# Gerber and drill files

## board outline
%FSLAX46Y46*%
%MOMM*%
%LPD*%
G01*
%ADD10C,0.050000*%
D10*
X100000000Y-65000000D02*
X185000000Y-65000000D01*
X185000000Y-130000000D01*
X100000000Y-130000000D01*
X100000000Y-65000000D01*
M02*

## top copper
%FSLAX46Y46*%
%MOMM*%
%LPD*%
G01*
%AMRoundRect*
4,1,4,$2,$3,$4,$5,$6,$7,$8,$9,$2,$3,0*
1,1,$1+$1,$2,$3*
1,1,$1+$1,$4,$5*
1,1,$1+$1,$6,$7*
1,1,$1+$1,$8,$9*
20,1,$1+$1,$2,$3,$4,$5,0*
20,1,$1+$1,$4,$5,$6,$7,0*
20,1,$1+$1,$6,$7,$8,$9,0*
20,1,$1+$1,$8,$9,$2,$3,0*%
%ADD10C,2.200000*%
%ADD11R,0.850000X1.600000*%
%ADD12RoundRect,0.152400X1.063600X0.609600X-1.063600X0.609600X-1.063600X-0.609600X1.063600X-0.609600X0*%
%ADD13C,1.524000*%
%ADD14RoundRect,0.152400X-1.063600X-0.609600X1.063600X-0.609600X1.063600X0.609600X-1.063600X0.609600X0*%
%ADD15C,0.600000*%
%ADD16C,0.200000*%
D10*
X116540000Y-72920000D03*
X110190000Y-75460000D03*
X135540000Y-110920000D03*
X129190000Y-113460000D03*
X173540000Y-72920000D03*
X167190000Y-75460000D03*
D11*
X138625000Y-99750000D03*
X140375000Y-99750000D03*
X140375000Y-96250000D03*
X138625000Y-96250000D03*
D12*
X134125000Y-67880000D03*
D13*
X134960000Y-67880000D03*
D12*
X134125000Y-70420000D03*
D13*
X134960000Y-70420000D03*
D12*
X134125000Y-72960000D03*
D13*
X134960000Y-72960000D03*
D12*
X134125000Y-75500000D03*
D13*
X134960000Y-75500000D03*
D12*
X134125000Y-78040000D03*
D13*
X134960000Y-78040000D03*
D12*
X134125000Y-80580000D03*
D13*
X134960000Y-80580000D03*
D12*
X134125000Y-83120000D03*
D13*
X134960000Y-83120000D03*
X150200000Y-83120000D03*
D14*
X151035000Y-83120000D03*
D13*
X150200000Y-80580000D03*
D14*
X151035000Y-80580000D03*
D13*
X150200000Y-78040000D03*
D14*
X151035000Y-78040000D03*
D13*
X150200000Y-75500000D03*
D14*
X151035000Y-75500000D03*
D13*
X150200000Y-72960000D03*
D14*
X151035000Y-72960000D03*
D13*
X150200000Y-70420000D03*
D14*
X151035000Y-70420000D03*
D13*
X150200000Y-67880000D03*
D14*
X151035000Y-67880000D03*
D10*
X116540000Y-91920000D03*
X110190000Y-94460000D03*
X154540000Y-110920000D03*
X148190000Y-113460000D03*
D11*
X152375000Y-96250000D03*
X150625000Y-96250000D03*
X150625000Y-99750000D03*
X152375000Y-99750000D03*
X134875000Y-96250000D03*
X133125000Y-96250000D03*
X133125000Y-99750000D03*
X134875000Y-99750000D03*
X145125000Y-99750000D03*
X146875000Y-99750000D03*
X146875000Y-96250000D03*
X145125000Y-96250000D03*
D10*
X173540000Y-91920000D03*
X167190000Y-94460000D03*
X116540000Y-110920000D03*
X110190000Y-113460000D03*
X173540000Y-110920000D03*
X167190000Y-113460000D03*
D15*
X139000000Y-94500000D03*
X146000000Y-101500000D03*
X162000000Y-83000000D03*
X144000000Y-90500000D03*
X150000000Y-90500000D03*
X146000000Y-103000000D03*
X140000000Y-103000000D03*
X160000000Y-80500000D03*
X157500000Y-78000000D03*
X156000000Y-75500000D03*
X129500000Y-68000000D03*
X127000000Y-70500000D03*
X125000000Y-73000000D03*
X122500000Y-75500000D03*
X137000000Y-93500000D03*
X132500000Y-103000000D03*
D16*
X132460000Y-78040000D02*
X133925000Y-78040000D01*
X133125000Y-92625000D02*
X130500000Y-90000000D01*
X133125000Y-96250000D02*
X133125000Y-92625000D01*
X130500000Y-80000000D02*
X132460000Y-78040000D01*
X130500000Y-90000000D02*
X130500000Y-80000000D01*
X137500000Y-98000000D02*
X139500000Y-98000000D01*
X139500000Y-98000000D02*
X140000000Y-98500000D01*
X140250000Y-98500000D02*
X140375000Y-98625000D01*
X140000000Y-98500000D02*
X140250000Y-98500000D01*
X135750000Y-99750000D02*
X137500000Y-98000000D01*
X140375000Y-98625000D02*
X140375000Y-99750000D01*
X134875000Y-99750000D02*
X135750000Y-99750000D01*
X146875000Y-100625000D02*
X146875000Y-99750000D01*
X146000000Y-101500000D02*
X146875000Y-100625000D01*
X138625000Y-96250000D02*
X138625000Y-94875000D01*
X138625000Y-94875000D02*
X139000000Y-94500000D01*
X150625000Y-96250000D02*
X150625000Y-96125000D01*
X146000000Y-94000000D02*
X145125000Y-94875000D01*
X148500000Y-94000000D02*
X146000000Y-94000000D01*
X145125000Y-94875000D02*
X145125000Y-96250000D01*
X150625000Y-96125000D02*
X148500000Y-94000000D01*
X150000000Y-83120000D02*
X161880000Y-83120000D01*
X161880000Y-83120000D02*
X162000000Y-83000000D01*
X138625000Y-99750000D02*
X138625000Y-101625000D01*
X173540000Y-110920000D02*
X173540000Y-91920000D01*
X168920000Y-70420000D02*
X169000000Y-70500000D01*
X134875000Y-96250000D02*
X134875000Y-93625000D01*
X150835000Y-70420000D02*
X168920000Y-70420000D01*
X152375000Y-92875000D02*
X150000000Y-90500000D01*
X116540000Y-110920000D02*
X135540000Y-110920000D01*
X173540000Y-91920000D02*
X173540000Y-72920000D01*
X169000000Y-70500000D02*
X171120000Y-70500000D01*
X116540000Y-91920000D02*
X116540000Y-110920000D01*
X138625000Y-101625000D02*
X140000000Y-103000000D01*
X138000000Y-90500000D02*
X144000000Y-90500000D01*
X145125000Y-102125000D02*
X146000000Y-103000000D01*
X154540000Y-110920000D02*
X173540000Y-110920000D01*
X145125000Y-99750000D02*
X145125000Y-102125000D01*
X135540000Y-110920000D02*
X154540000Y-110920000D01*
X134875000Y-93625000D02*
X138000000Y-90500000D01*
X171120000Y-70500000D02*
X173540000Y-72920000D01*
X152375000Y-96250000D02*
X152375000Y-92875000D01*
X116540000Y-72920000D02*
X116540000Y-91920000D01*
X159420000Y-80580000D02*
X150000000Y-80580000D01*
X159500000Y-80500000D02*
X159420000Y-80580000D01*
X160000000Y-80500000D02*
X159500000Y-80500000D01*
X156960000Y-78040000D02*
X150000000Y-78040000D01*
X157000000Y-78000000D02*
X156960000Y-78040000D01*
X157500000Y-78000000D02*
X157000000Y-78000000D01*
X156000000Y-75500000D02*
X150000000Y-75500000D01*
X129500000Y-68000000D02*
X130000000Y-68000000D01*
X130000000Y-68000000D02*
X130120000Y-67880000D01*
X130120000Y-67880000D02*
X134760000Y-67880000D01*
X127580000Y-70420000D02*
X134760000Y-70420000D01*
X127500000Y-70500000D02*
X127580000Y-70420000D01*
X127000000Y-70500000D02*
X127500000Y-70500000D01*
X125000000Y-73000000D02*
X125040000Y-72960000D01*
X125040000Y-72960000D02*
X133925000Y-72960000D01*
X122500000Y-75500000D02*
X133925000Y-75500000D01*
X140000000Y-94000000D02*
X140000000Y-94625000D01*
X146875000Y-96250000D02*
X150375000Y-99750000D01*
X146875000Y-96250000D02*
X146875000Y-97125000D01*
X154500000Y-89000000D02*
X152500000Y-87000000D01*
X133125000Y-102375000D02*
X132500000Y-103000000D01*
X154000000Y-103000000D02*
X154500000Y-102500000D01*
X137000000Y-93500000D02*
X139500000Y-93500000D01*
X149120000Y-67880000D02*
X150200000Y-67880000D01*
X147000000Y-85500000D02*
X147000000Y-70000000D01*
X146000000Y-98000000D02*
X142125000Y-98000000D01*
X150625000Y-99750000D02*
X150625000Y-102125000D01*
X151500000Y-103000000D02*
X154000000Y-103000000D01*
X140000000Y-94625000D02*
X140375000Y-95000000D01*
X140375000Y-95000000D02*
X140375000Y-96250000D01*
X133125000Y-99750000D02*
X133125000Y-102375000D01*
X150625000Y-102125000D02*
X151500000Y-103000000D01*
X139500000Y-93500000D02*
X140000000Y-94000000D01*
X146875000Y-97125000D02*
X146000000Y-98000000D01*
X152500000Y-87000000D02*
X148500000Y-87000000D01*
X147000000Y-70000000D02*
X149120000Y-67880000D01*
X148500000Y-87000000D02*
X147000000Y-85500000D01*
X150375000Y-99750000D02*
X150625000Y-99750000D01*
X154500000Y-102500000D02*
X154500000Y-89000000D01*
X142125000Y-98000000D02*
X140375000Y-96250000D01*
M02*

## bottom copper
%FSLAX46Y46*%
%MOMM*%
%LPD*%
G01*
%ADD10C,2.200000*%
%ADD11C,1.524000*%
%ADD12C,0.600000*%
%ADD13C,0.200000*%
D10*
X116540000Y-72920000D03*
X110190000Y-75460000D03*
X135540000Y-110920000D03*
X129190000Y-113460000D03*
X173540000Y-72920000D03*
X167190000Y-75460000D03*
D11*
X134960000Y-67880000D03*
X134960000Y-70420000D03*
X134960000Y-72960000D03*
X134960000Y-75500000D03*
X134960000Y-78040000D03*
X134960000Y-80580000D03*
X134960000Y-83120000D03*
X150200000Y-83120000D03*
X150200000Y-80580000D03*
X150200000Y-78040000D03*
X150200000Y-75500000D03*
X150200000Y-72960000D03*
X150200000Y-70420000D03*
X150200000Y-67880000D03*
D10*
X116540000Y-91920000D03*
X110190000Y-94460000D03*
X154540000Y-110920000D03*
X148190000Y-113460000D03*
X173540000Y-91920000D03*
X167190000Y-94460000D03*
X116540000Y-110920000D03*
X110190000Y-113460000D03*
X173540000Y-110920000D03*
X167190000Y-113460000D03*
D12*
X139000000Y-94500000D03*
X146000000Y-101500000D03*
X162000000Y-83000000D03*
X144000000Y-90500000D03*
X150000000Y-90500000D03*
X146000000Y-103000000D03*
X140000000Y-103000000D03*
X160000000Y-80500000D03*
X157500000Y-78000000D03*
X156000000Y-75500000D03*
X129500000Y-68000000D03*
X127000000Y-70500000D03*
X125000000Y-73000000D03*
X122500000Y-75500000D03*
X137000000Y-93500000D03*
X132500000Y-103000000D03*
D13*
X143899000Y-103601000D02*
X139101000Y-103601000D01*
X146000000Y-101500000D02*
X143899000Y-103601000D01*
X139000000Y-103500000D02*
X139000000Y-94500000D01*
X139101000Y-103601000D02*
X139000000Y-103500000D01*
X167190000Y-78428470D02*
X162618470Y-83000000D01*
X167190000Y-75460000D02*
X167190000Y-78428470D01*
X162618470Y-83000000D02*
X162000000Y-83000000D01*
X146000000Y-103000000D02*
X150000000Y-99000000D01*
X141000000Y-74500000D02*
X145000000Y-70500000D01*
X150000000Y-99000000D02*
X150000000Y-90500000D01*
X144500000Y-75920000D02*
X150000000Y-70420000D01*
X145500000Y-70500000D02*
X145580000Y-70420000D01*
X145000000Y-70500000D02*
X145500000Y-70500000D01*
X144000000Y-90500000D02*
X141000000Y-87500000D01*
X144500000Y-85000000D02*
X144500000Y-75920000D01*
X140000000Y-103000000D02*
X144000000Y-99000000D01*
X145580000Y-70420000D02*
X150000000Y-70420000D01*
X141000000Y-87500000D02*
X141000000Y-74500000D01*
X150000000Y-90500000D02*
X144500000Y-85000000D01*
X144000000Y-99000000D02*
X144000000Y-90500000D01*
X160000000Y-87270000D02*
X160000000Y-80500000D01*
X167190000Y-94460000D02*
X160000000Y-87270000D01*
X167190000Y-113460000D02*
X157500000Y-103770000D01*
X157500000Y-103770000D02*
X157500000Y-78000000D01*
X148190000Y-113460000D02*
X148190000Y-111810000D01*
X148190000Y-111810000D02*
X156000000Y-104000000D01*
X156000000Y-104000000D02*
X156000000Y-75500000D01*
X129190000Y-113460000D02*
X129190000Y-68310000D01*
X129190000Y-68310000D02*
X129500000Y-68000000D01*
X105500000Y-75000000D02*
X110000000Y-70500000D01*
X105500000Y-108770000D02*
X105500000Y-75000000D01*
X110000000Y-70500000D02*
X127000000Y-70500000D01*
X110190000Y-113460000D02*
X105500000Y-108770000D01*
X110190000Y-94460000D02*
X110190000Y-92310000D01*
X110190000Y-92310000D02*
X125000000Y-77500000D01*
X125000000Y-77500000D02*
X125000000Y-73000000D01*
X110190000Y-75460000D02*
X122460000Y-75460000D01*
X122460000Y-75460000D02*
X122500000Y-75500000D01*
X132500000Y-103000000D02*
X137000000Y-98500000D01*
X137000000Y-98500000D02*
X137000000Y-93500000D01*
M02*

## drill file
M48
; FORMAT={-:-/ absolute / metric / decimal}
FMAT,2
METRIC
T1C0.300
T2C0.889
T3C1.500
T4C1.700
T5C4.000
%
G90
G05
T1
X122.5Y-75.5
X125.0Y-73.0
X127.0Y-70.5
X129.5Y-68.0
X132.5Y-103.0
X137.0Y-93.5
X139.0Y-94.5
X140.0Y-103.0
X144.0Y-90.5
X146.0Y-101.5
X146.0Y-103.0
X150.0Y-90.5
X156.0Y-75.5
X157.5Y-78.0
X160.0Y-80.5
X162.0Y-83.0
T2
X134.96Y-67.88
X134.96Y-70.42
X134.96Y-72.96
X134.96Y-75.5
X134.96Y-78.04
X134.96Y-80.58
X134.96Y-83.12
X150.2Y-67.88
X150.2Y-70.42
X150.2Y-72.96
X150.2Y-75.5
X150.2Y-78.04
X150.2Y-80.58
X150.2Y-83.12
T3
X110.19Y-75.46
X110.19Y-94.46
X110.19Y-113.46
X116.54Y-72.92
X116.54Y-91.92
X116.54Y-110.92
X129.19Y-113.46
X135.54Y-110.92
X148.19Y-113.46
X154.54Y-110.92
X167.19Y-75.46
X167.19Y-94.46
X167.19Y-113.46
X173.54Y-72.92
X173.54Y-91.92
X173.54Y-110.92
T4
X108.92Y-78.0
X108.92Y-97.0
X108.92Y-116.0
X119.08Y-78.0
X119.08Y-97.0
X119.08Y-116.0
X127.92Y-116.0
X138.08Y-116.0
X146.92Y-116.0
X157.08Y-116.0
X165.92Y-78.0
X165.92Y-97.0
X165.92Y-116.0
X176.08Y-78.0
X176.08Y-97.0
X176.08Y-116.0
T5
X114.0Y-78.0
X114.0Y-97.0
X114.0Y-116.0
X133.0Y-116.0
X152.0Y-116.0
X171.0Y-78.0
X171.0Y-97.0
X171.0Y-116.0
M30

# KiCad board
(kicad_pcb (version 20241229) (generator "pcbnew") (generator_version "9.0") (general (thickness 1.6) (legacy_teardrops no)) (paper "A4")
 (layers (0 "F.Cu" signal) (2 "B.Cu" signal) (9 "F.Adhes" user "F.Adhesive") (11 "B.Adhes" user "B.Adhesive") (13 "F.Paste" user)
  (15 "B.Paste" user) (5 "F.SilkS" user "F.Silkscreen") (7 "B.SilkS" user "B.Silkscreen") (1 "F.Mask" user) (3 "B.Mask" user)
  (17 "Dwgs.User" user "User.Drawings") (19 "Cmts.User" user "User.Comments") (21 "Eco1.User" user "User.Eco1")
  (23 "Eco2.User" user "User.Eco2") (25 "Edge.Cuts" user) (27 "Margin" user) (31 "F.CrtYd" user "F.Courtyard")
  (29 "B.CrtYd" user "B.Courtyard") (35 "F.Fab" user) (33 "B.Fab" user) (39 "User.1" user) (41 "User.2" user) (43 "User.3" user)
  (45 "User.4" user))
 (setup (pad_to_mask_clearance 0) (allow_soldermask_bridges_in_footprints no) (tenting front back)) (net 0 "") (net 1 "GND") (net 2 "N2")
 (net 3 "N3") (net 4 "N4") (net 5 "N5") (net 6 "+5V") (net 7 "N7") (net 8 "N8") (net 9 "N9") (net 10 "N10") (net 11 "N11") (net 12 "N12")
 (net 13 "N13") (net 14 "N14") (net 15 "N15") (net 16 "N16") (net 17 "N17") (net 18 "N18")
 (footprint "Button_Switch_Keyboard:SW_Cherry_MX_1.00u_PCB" (layer "F.Cu") (at 116.54 72.92)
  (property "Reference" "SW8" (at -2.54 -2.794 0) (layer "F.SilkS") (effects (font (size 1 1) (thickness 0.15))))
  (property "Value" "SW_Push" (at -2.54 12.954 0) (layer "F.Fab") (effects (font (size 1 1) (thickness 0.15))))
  (pad "" np_thru_hole circle (at -7.62 5.08) (size 1.7 1.7) (drill 1.7) (layers "*.Cu" "*.Mask"))
  (pad "" np_thru_hole circle (at -2.54 5.08) (size 4 4) (drill 4) (layers "*.Cu" "*.Mask"))
  (pad "" np_thru_hole circle (at 2.54 5.08) (size 1.7 1.7) (drill 1.7) (layers "*.Cu" "*.Mask"))
  (pad "1" thru_hole circle (at 0 0) (size 2.2 2.2) (drill 1.5) (layers "*.Cu" "*.Mask") (remove_unused_layers no) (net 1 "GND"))
  (pad "2" thru_hole circle (at -6.35 2.54) (size 2.2 2.2) (drill 1.5) (layers "*.Cu" "*.Mask") (remove_unused_layers no) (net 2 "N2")))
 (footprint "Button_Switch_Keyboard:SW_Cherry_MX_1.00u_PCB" (layer "F.Cu") (at 135.54 110.92)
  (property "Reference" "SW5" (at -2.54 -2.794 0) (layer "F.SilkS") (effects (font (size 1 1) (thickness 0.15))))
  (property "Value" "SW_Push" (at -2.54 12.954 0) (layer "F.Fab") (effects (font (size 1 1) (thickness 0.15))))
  (pad "" np_thru_hole circle (at -7.62 5.08) (size 1.7 1.7) (drill 1.7) (layers "*.Cu" "*.Mask"))
  (pad "" np_thru_hole circle (at -2.54 5.08) (size 4 4) (drill 4) (layers "*.Cu" "*.Mask"))
  (pad "" np_thru_hole circle (at 2.54 5.08) (size 1.7 1.7) (drill 1.7) (layers "*.Cu" "*.Mask"))
  (pad "1" thru_hole circle (at 0 0) (size 2.2 2.2) (drill 1.5) (layers "*.Cu" "*.Mask") (remove_unused_layers no) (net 1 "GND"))
  (pad "2" thru_hole circle (at -6.35 2.54) (size 2.2 2.2) (drill 1.5) (layers "*.Cu" "*.Mask") (remove_unused_layers no) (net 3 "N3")))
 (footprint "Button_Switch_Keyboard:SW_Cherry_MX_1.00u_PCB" (layer "F.Cu") (at 173.54 72.92)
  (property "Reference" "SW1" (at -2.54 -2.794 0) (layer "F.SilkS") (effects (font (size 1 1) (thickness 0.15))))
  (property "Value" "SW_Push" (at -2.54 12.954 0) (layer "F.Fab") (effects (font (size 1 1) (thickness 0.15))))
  (pad "" np_thru_hole circle (at -7.62 5.08) (size 1.7 1.7) (drill 1.7) (layers "*.Cu" "*.Mask"))
  (pad "" np_thru_hole circle (at -2.54 5.08) (size 4 4) (drill 4) (layers "*.Cu" "*.Mask"))
  (pad "" np_thru_hole circle (at 2.54 5.08) (size 1.7 1.7) (drill 1.7) (layers "*.Cu" "*.Mask"))
  (pad "1" thru_hole circle (at 0 0) (size 2.2 2.2) (drill 1.5) (layers "*.Cu" "*.Mask") (remove_unused_layers no) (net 1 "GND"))
  (pad "2" thru_hole circle (at -6.35 2.54) (size 2.2 2.2) (drill 1.5) (layers "*.Cu" "*.Mask") (remove_unused_layers no) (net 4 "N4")))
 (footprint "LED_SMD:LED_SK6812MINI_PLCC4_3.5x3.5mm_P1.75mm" (layer "F.Cu") (at 139.5 98 90)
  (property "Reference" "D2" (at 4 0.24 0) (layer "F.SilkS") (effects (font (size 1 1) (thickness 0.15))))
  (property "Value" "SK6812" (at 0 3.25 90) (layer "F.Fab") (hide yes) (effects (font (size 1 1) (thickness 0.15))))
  (pad "1" smd rect (at -1.75 -0.875 90) (size 1.6 0.85) (layers "F.Cu" "F.Mask" "F.Paste") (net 1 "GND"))
  (pad "2" smd rect (at -1.75 0.875 90) (size 1.6 0.85) (layers "F.Cu" "F.Mask" "F.Paste") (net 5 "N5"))
  (pad "3" smd rect (at 1.75 0.875 90) (size 1.6 0.85) (layers "F.Cu" "F.Mask" "F.Paste") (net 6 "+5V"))
  (pad "4" smd rect (at 1.75 -0.875 90) (size 1.6 0.85) (layers "F.Cu" "F.Mask" "F.Paste") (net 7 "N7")))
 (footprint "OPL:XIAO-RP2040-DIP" (layer "F.Cu") (at 142.58 75.5)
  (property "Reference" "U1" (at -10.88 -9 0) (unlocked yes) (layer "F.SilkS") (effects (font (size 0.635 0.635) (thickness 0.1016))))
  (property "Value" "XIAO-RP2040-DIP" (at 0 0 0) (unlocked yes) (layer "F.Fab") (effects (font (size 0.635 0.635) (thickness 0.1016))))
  (pad "1" smd roundrect (at -8.455 -7.62 180) (size 2.432 1.524) (layers "F.Cu" "F.Mask") (roundrect_rratio 0.1) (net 3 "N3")
   (thermal_bridge_angle 45))
  (pad "1" thru_hole circle (at -7.62 -7.62 180) (size 1.524 1.524) (drill 0.889) (layers "*.Cu" "*.Mask") (remove_unused_layers no)
   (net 3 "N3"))
  (pad "2" smd roundrect (at -8.455 -5.08 180) (size 2.432 1.524) (layers "F.Cu" "F.Mask") (roundrect_rratio 0.1) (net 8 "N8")
   (thermal_bridge_angle 45))
  (pad "2" thru_hole circle (at -7.62 -5.08 180) (size 1.524 1.524) (drill 0.889) (layers "*.Cu" "*.Mask") (remove_unused_layers no)
   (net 8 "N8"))
  (pad "3" smd roundrect (at -8.455 -2.54 180) (size 2.432 1.524) (layers "F.Cu" "F.Mask") (roundrect_rratio 0.1) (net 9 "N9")
   (thermal_bridge_angle 45))
  (pad "3" thru_hole circle (at -7.62 -2.54 180) (size 1.524 1.524) (drill 0.889) (layers "*.Cu" "*.Mask") (remove_unused_layers no)
   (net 9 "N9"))
  (pad "4" smd roundrect (at -8.455 0 180) (size 2.432 1.524) (layers "F.Cu" "F.Mask") (roundrect_rratio 0.1) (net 2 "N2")
   (thermal_bridge_angle 45))
  (pad "4" thru_hole circle (at -7.62 0 180) (size 1.524 1.524) (drill 0.889) (layers "*.Cu" "*.Mask") (remove_unused_layers no)
   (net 2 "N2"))
  (pad "5" smd roundrect (at -8.455 2.54 180) (size 2.432 1.524) (layers "F.Cu" "F.Mask") (roundrect_rratio 0.1) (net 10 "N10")
   (thermal_bridge_angle 45))
  (pad "5" thru_hole circle (at -7.62 2.54 180) (size 1.524 1.524) (drill 0.889) (layers "*.Cu" "*.Mask") (remove_unused_layers no)
   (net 10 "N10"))
  (pad "6" smd roundrect (at -8.455 5.08 180) (size 2.432 1.524) (layers "F.Cu" "F.Mask") (roundrect_rratio 0.1) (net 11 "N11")
   (thermal_bridge_angle 45))
  (pad "6" thru_hole circle (at -7.62 5.08 180) (size 1.524 1.524) (drill 0.889) (layers "*.Cu" "*.Mask") (remove_unused_layers no)
   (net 11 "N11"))
  (pad "7" smd roundrect (at -8.455 7.62 180) (size 2.432 1.524) (layers "F.Cu" "F.Mask") (roundrect_rratio 0.1) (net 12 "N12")
   (thermal_bridge_angle 45))
  (pad "7" thru_hole circle (at -7.62 7.62 180) (size 1.524 1.524) (drill 0.889) (layers "*.Cu" "*.Mask") (remove_unused_layers no)
   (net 12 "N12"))
  (pad "8" thru_hole circle (at 7.62 7.62) (size 1.524 1.524) (drill 0.889) (layers "*.Cu" "*.Mask") (remove_unused_layers no) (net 4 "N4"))
  (pad "8" smd roundrect (at 8.455 7.62) (size 2.432 1.524) (layers "F.Cu" "F.Mask") (roundrect_rratio 0.1) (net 4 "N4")
   (thermal_bridge_angle 45))
  (pad "9" thru_hole circle (at 7.62 5.08) (size 1.524 1.524) (drill 0.889) (layers "*.Cu" "*.Mask") (remove_unused_layers no)
   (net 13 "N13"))
  (pad "9" smd roundrect (at 8.455 5.08) (size 2.432 1.524) (layers "F.Cu" "F.Mask") (roundrect_rratio 0.1) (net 13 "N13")
   (thermal_bridge_angle 45))
  (pad "10" thru_hole circle (at 7.62 2.54) (size 1.524 1.524) (drill 0.889) (layers "*.Cu" "*.Mask") (remove_unused_layers no)
   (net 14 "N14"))
  (pad "10" smd roundrect (at 8.455 2.54) (size 2.432 1.524) (layers "F.Cu" "F.Mask") (roundrect_rratio 0.1) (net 14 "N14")
   (thermal_bridge_angle 45))
  (pad "11" thru_hole circle (at 7.62 0) (size 1.524 1.524) (drill 0.889) (layers "*.Cu" "*.Mask") (remove_unused_layers no) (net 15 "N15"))
  (pad "11" smd roundrect (at 8.455 0) (size 2.432 1.524) (layers "F.Cu" "F.Mask") (roundrect_rratio 0.1) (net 15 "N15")
   (thermal_bridge_angle 45))
  (pad "12" thru_hole circle (at 7.62 -2.54) (size 1.524 1.524) (drill 0.889) (layers "*.Cu" "*.Mask") (remove_unused_layers no)
   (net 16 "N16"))
  (pad "12" smd roundrect (at 8.455 -2.54) (size 2.432 1.524) (layers "F.Cu" "F.Mask") (roundrect_rratio 0.1) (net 16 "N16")
   (thermal_bridge_angle 45))
  (pad "13" thru_hole circle (at 7.62 -5.08) (size 1.524 1.524) (drill 0.889) (layers "*.Cu" "*.Mask") (remove_unused_layers no)
   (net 1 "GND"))
  (pad "13" smd roundrect (at 8.455 -5.08) (size 2.432 1.524) (layers "F.Cu" "F.Mask") (roundrect_rratio 0.1) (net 1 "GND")
   (thermal_bridge_angle 45))
  (pad "14" thru_hole circle (at 7.62 -7.62) (size 1.524 1.524) (drill 0.889) (layers "*.Cu" "*.Mask") (remove_unused_layers no)
   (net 6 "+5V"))
  (pad "14" smd roundrect (at 8.455 -7.62) (size 2.432 1.524) (layers "F.Cu" "F.Mask") (roundrect_rratio 0.1) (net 6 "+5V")
   (thermal_bridge_angle 45)))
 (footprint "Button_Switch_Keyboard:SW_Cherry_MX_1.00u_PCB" (layer "F.Cu") (at 116.54 91.92)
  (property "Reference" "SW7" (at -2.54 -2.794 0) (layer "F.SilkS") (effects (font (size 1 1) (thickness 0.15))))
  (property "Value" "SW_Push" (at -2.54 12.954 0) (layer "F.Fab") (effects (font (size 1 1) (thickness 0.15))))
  (pad "" np_thru_hole circle (at -7.62 5.08) (size 1.7 1.7) (drill 1.7) (layers "*.Cu" "*.Mask"))
  (pad "" np_thru_hole circle (at -2.54 5.08) (size 4 4) (drill 4) (layers "*.Cu" "*.Mask"))
  (pad "" np_thru_hole circle (at 2.54 5.08) (size 1.7 1.7) (drill 1.7) (layers "*.Cu" "*.Mask"))
  (pad "1" thru_hole circle (at 0 0) (size 2.2 2.2) (drill 1.5) (layers "*.Cu" "*.Mask") (remove_unused_layers no) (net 1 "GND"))
  (pad "2" thru_hole circle (at -6.35 2.54) (size 2.2 2.2) (drill 1.5) (layers "*.Cu" "*.Mask") (remove_unused_layers no) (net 9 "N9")))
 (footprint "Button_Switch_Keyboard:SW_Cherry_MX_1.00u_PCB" (layer "F.Cu") (at 154.54 110.92)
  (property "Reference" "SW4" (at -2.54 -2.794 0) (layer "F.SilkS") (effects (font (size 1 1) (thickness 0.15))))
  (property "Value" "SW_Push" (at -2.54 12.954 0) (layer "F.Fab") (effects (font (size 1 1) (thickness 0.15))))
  (pad "" np_thru_hole circle (at -7.62 5.08) (size 1.7 1.7) (drill 1.7) (layers "*.Cu" "*.Mask"))
  (pad "" np_thru_hole circle (at -2.54 5.08) (size 4 4) (drill 4) (layers "*.Cu" "*.Mask"))
  (pad "" np_thru_hole circle (at 2.54 5.08) (size 1.7 1.7) (drill 1.7) (layers "*.Cu" "*.Mask"))
  (pad "1" thru_hole circle (at 0 0) (size 2.2 2.2) (drill 1.5) (layers "*.Cu" "*.Mask") (remove_unused_layers no) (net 1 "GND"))
  (pad "2" thru_hole circle (at -6.35 2.54) (size 2.2 2.2) (drill 1.5) (layers "*.Cu" "*.Mask") (remove_unused_layers no) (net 15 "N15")))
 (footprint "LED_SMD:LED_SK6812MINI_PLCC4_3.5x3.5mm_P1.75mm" (layer "F.Cu") (at 151.5 98 -90)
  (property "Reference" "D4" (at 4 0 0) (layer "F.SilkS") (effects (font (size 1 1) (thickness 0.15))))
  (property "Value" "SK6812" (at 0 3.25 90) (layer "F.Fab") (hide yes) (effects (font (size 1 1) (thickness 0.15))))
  (pad "1" smd rect (at -1.75 -0.875 270) (size 1.6 0.85) (layers "F.Cu" "F.Mask" "F.Paste") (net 1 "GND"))
  (pad "2" smd rect (at -1.75 0.875 270) (size 1.6 0.85) (layers "F.Cu" "F.Mask" "F.Paste") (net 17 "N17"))
  (pad "3" smd rect (at 1.75 0.875 270) (size 1.6 0.85) (layers "F.Cu" "F.Mask" "F.Paste") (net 6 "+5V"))
  (pad "4" smd rect (at 1.75 -0.875 270) (size 1.6 0.85) (layers "F.Cu" "F.Mask" "F.Paste") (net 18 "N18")))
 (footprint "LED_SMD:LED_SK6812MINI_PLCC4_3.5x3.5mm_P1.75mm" (layer "F.Cu") (at 134 98 -90)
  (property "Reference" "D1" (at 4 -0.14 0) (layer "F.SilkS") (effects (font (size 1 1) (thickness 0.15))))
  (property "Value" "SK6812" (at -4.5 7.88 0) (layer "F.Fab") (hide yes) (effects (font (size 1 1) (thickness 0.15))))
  (pad "1" smd rect (at -1.75 -0.875 270) (size 1.6 0.85) (layers "F.Cu" "F.Mask" "F.Paste") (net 1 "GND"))
  (pad "2" smd rect (at -1.75 0.875 270) (size 1.6 0.85) (layers "F.Cu" "F.Mask" "F.Paste") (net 10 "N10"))
  (pad "3" smd rect (at 1.75 0.875 270) (size 1.6 0.85) (layers "F.Cu" "F.Mask" "F.Paste") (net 6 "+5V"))
  (pad "4" smd rect (at 1.75 -0.875 270) (size 1.6 0.85) (layers "F.Cu" "F.Mask" "F.Paste") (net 5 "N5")))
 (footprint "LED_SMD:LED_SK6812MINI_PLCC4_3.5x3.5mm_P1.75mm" (layer "F.Cu") (at 146 98 90)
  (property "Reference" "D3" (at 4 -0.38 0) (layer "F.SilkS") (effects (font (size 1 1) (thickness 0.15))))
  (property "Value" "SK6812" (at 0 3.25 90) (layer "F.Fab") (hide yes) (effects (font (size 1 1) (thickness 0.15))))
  (pad "1" smd rect (at -1.75 -0.875 90) (size 1.6 0.85) (layers "F.Cu" "F.Mask" "F.Paste") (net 1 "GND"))
  (pad "2" smd rect (at -1.75 0.875 90) (size 1.6 0.85) (layers "F.Cu" "F.Mask" "F.Paste") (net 7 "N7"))
  (pad "3" smd rect (at 1.75 0.875 90) (size 1.6 0.85) (layers "F.Cu" "F.Mask" "F.Paste") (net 6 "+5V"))
  (pad "4" smd rect (at 1.75 -0.875 90) (size 1.6 0.85) (layers "F.Cu" "F.Mask" "F.Paste") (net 17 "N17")))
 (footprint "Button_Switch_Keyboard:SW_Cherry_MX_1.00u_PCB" (layer "F.Cu") (at 173.54 91.92)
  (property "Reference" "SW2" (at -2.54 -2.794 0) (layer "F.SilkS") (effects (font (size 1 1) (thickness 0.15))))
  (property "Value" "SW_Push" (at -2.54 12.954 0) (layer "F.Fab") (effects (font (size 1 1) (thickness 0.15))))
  (pad "" np_thru_hole circle (at -7.62 5.08) (size 1.7 1.7) (drill 1.7) (layers "*.Cu" "*.Mask"))
  (pad "" np_thru_hole circle (at -2.54 5.08) (size 4 4) (drill 4) (layers "*.Cu" "*.Mask"))
  (pad "" np_thru_hole circle (at 2.54 5.08) (size 1.7 1.7) (drill 1.7) (layers "*.Cu" "*.Mask"))
  (pad "1" thru_hole circle (at 0 0) (size 2.2 2.2) (drill 1.5) (layers "*.Cu" "*.Mask") (remove_unused_layers no) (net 1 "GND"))
  (pad "2" thru_hole circle (at -6.35 2.54) (size 2.2 2.2) (drill 1.5) (layers "*.Cu" "*.Mask") (remove_unused_layers no) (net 13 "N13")))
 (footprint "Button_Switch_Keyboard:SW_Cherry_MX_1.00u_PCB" (layer "F.Cu") (at 116.54 110.92)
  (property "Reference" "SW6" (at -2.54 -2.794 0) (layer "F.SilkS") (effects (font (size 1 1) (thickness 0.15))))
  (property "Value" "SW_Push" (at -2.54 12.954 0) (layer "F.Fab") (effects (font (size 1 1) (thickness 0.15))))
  (pad "" np_thru_hole circle (at -7.62 5.08) (size 1.7 1.7) (drill 1.7) (layers "*.Cu" "*.Mask"))
  (pad "" np_thru_hole circle (at -2.54 5.08) (size 4 4) (drill 4) (layers "*.Cu" "*.Mask"))
  (pad "" np_thru_hole circle (at 2.54 5.08) (size 1.7 1.7) (drill 1.7) (layers "*.Cu" "*.Mask"))
  (pad "1" thru_hole circle (at 0 0) (size 2.2 2.2) (drill 1.5) (layers "*.Cu" "*.Mask") (remove_unused_layers no) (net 1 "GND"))
  (pad "2" thru_hole circle (at -6.35 2.54) (size 2.2 2.2) (drill 1.5) (layers "*.Cu" "*.Mask") (remove_unused_layers no) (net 8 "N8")))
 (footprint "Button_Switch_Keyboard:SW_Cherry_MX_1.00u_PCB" (layer "F.Cu") (at 173.54 110.92)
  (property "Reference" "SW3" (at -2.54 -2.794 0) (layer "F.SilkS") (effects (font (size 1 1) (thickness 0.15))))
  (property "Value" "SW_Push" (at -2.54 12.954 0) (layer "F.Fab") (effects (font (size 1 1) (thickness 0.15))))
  (pad "" np_thru_hole circle (at -7.62 5.08) (size 1.7 1.7) (drill 1.7) (layers "*.Cu" "*.Mask"))
  (pad "" np_thru_hole circle (at -2.54 5.08) (size 4 4) (drill 4) (layers "*.Cu" "*.Mask"))
  (pad "" np_thru_hole circle (at 2.54 5.08) (size 1.7 1.7) (drill 1.7) (layers "*.Cu" "*.Mask"))
  (pad "1" thru_hole circle (at 0 0) (size 2.2 2.2) (drill 1.5) (layers "*.Cu" "*.Mask") (remove_unused_layers no) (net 1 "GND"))
  (pad "2" thru_hole circle (at -6.35 2.54) (size 2.2 2.2) (drill 1.5) (layers "*.Cu" "*.Mask") (remove_unused_layers no) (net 14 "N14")))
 (gr_rect (start 100 65) (end 185 130) (stroke (width 0.05) (type default)) (fill no) (layer "Edge.Cuts"))
 (segment (start 132.46 78.04) (end 133.925 78.04) (width 0.2) (layer "F.Cu") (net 10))
 (segment (start 133.125 92.625) (end 130.5 90) (width 0.2) (layer "F.Cu") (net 10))
 (segment (start 133.125 96.25) (end 133.125 92.625) (width 0.2) (layer "F.Cu") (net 10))
 (segment (start 130.5 80) (end 132.46 78.04) (width 0.2) (layer "F.Cu") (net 10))
 (segment (start 130.5 90) (end 130.5 80) (width 0.2) (layer "F.Cu") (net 10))
 (segment (start 137.5 98) (end 139.5 98) (width 0.2) (layer "F.Cu") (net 5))
 (segment (start 139.5 98) (end 140 98.5) (width 0.2) (layer "F.Cu") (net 5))
 (segment (start 140.25 98.5) (end 140.375 98.625) (width 0.2) (layer "F.Cu") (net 5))
 (segment (start 140 98.5) (end 140.25 98.5) (width 0.2) (layer "F.Cu") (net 5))
 (segment (start 135.75 99.75) (end 137.5 98) (width 0.2) (layer "F.Cu") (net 5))
 (segment (start 140.375 98.625) (end 140.375 99.75) (width 0.2) (layer "F.Cu") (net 5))
 (segment (start 134.875 99.75) (end 135.75 99.75) (width 0.2) (layer "F.Cu") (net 5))
 (segment (start 146.875 100.625) (end 146.875 99.75) (width 0.2) (layer "F.Cu") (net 7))
 (segment (start 146 101.5) (end 146.875 100.625) (width 0.2) (layer "F.Cu") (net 7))
 (segment (start 138.625 96.25) (end 138.625 94.875) (width 0.2) (layer "F.Cu") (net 7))
 (segment (start 138.625 94.875) (end 139 94.5) (width 0.2) (layer "F.Cu") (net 7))
 (via (at 139 94.5) (size 0.6) (drill 0.3) (layers "F.Cu" "B.Cu") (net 7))
 (via (at 146 101.5) (size 0.6) (drill 0.3) (layers "F.Cu" "B.Cu") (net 7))
 (segment (start 143.899 103.601) (end 139.101 103.601) (width 0.2) (layer "B.Cu") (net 7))
 (segment (start 146 101.5) (end 143.899 103.601) (width 0.2) (layer "B.Cu") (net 7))
 (segment (start 139 103.5) (end 139 94.5) (width 0.2) (layer "B.Cu") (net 7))
 (segment (start 139.101 103.601) (end 139 103.5) (width 0.2) (layer "B.Cu") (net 7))
 (segment (start 150.625 96.25) (end 150.625 96.125) (width 0.2) (layer "F.Cu") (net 17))
 (segment (start 146 94) (end 145.125 94.875) (width 0.2) (layer "F.Cu") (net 17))
 (segment (start 148.5 94) (end 146 94) (width 0.2) (layer "F.Cu") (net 17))
 (segment (start 145.125 94.875) (end 145.125 96.25) (width 0.2) (layer "F.Cu") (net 17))
 (segment (start 150.625 96.125) (end 148.5 94) (width 0.2) (layer "F.Cu") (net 17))
 (segment (start 150 83.12) (end 161.88 83.12) (width 0.2) (layer "F.Cu") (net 4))
 (segment (start 161.88 83.12) (end 162 83) (width 0.2) (layer "F.Cu") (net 4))
 (via (at 162 83) (size 0.6) (drill 0.3) (layers "F.Cu" "B.Cu") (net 4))
 (segment (start 167.19 78.42847) (end 162.61847 83) (width 0.2) (layer "B.Cu") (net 4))
 (segment (start 167.19 75.46) (end 167.19 78.42847) (width 0.2) (layer "B.Cu") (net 4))
 (segment (start 162.61847 83) (end 162 83) (width 0.2) (layer "B.Cu") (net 4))
 (segment (start 138.625 99.75) (end 138.625 101.625) (width 0.2) (layer "F.Cu") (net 1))
 (segment (start 173.54 110.92) (end 173.54 91.92) (width 0.2) (layer "F.Cu") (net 1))
 (segment (start 168.92 70.42) (end 169 70.5) (width 0.2) (layer "F.Cu") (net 1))
 (segment (start 134.875 96.25) (end 134.875 93.625) (width 0.2) (layer "F.Cu") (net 1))
 (segment (start 150.835 70.42) (end 168.92 70.42) (width 0.2) (layer "F.Cu") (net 1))
 (segment (start 152.375 92.875) (end 150 90.5) (width 0.2) (layer "F.Cu") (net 1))
 (segment (start 116.54 110.92) (end 135.54 110.92) (width 0.2) (layer "F.Cu") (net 1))
 (segment (start 173.54 91.92) (end 173.54 72.92) (width 0.2) (layer "F.Cu") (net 1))
 (segment (start 169 70.5) (end 171.12 70.5) (width 0.2) (layer "F.Cu") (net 1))
 (segment (start 116.54 91.92) (end 116.54 110.92) (width 0.2) (layer "F.Cu") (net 1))
 (segment (start 138.625 101.625) (end 140 103) (width 0.2) (layer "F.Cu") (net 1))
 (segment (start 138 90.5) (end 144 90.5) (width 0.2) (layer "F.Cu") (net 1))
 (segment (start 145.125 102.125) (end 146 103) (width 0.2) (layer "F.Cu") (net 1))
 (segment (start 154.54 110.92) (end 173.54 110.92) (width 0.2) (layer "F.Cu") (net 1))
 (segment (start 145.125 99.75) (end 145.125 102.125) (width 0.2) (layer "F.Cu") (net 1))
 (segment (start 135.54 110.92) (end 154.54 110.92) (width 0.2) (layer "F.Cu") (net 1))
 (segment (start 134.875 93.625) (end 138 90.5) (width 0.2) (layer "F.Cu") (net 1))
 (segment (start 171.12 70.5) (end 173.54 72.92) (width 0.2) (layer "F.Cu") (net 1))
 (segment (start 152.375 96.25) (end 152.375 92.875) (width 0.2) (layer "F.Cu") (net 1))
 (segment (start 116.54 72.92) (end 116.54 91.92) (width 0.2) (layer "F.Cu") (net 1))
 (via (at 144 90.5) (size 0.6) (drill 0.3) (layers "F.Cu" "B.Cu") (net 1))
 (via (at 150 90.5) (size 0.6) (drill 0.3) (layers "F.Cu" "B.Cu") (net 1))
 (via (at 146 103) (size 0.6) (drill 0.3) (layers "F.Cu" "B.Cu") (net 1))
 (via (at 140 103) (size 0.6) (drill 0.3) (layers "F.Cu" "B.Cu") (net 1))
 (segment (start 146 103) (end 150 99) (width 0.2) (layer "B.Cu") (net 1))
 (segment (start 141 74.5) (end 145 70.5) (width 0.2) (layer "B.Cu") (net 1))
 (segment (start 150 99) (end 150 90.5) (width 0.2) (layer "B.Cu") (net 1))
 (segment (start 144.5 75.92) (end 150 70.42) (width 0.2) (layer "B.Cu") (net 1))
 (segment (start 145.5 70.5) (end 145.58 70.42) (width 0.2) (layer "B.Cu") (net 1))
 (segment (start 145 70.5) (end 145.5 70.5) (width 0.2) (layer "B.Cu") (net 1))
 (segment (start 144 90.5) (end 141 87.5) (width 0.2) (layer "B.Cu") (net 1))
 (segment (start 144.5 85) (end 144.5 75.92) (width 0.2) (layer "B.Cu") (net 1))
 (segment (start 140 103) (end 144 99) (width 0.2) (layer "B.Cu") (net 1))
 (segment (start 145.58 70.42) (end 150 70.42) (width 0.2) (layer "B.Cu") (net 1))
 (segment (start 141 87.5) (end 141 74.5) (width 0.2) (layer "B.Cu") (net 1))
 (segment (start 150 90.5) (end 144.5 85) (width 0.2) (layer "B.Cu") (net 1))
 (segment (start 144 99) (end 144 90.5) (width 0.2) (layer "B.Cu") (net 1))
 (segment (start 159.42 80.58) (end 150 80.58) (width 0.2) (layer "F.Cu") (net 13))
 (segment (start 159.5 80.5) (end 159.42 80.58) (width 0.2) (layer "F.Cu") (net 13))
 (segment (start 160 80.5) (end 159.5 80.5) (width 0.2) (layer "F.Cu") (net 13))
 (via (at 160 80.5) (size 0.6) (drill 0.3) (layers "F.Cu" "B.Cu") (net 13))
 (segment (start 160 87.27) (end 160 80.5) (width 0.2) (layer "B.Cu") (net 13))
 (segment (start 167.19 94.46) (end 160 87.27) (width 0.2) (layer "B.Cu") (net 13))
 (segment (start 156.96 78.04) (end 150 78.04) (width 0.2) (layer "F.Cu") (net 14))
 (segment (start 157 78) (end 156.96 78.04) (width 0.2) (layer "F.Cu") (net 14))
 (segment (start 157.5 78) (end 157 78) (width 0.2) (layer "F.Cu") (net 14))
 (via (at 157.5 78) (size 0.6) (drill 0.3) (layers "F.Cu" "B.Cu") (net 14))
 (segment (start 167.19 113.46) (end 157.5 103.77) (width 0.2) (layer "B.Cu") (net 14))
 (segment (start 157.5 103.77) (end 157.5 78) (width 0.2) (layer "B.Cu") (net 14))
 (segment (start 156 75.5) (end 150 75.5) (width 0.2) (layer "F.Cu") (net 15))
 (via (at 156 75.5) (size 0.6) (drill 0.3) (layers "F.Cu" "B.Cu") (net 15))
 (segment (start 148.19 113.46) (end 148.19 111.81) (width 0.2) (layer "B.Cu") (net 15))
 (segment (start 148.19 111.81) (end 156 104) (width 0.2) (layer "B.Cu") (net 15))
 (segment (start 156 104) (end 156 75.5) (width 0.2) (layer "B.Cu") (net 15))
 (segment (start 129.5 68) (end 130 68) (width 0.2) (layer "F.Cu") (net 3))
 (segment (start 130 68) (end 130.12 67.88) (width 0.2) (layer "F.Cu") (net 3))
 (segment (start 130.12 67.88) (end 134.76 67.88) (width 0.2) (layer "F.Cu") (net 3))
 (via (at 129.5 68) (size 0.6) (drill 0.3) (layers "F.Cu" "B.Cu") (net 3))
 (segment (start 129.19 113.46) (end 129.19 68.31) (width 0.2) (layer "B.Cu") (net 3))
 (segment (start 129.19 68.31) (end 129.5 68) (width 0.2) (layer "B.Cu") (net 3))
 (segment (start 127.58 70.42) (end 134.76 70.42) (width 0.2) (layer "F.Cu") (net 8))
 (segment (start 127.5 70.5) (end 127.58 70.42) (width 0.2) (layer "F.Cu") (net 8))
 (segment (start 127 70.5) (end 127.5 70.5) (width 0.2) (layer "F.Cu") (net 8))
 (via (at 127 70.5) (size 0.6) (drill 0.3) (layers "F.Cu" "B.Cu") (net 8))
 (segment (start 105.5 75) (end 110 70.5) (width 0.2) (layer "B.Cu") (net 8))
 (segment (start 105.5 108.77) (end 105.5 75) (width 0.2) (layer "B.Cu") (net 8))
 (segment (start 110 70.5) (end 127 70.5) (width 0.2) (layer "B.Cu") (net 8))
 (segment (start 110.19 113.46) (end 105.5 108.77) (width 0.2) (layer "B.Cu") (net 8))
 (segment (start 125 73) (end 125.04 72.96) (width 0.2) (layer "F.Cu") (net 9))
 (segment (start 125.04 72.96) (end 133.925 72.96) (width 0.2) (layer "F.Cu") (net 9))
 (via (at 125 73) (size 0.6) (drill 0.3) (layers "F.Cu" "B.Cu") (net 9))
 (segment (start 110.19 94.46) (end 110.19 92.31) (width 0.2) (layer "B.Cu") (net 9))
 (segment (start 110.19 92.31) (end 125 77.5) (width 0.2) (layer "B.Cu") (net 9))
 (segment (start 125 77.5) (end 125 73) (width 0.2) (layer "B.Cu") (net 9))
 (segment (start 122.5 75.5) (end 133.925 75.5) (width 0.2) (layer "F.Cu") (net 2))
 (via (at 122.5 75.5) (size 0.6) (drill 0.3) (layers "F.Cu" "B.Cu") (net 2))
 (segment (start 110.19 75.46) (end 122.46 75.46) (width 0.2) (layer "B.Cu") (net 2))
 (segment (start 122.46 75.46) (end 122.5 75.5) (width 0.2) (layer "B.Cu") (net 2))
 (segment (start 140 94) (end 140 94.625) (width 0.2) (layer "F.Cu") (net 6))
 (segment (start 146.875 96.25) (end 150.375 99.75) (width 0.2) (layer "F.Cu") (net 6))
 (segment (start 146.875 96.25) (end 146.875 97.125) (width 0.2) (layer "F.Cu") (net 6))
 (segment (start 154.5 89) (end 152.5 87) (width 0.2) (layer "F.Cu") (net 6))
 (segment (start 133.125 102.375) (end 132.5 103) (width 0.2) (layer "F.Cu") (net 6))
 (segment (start 154 103) (end 154.5 102.5) (width 0.2) (layer "F.Cu") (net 6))
 (segment (start 137 93.5) (end 139.5 93.5) (width 0.2) (layer "F.Cu") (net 6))
 (segment (start 149.12 67.88) (end 150.2 67.88) (width 0.2) (layer "F.Cu") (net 6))
 (segment (start 147 85.5) (end 147 70) (width 0.2) (layer "F.Cu") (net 6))
 (segment (start 146 98) (end 142.125 98) (width 0.2) (layer "F.Cu") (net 6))
 (segment (start 150.625 99.75) (end 150.625 102.125) (width 0.2) (layer "F.Cu") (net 6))
 (segment (start 151.5 103) (end 154 103) (width 0.2) (layer "F.Cu") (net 6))
 (segment (start 140 94.625) (end 140.375 95) (width 0.2) (layer "F.Cu") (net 6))
 (segment (start 140.375 95) (end 140.375 96.25) (width 0.2) (layer "F.Cu") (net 6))
 (segment (start 133.125 99.75) (end 133.125 102.375) (width 0.2) (layer "F.Cu") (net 6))
 (segment (start 150.625 102.125) (end 151.5 103) (width 0.2) (layer "F.Cu") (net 6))
 (segment (start 139.5 93.5) (end 140 94) (width 0.2) (layer "F.Cu") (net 6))
 (segment (start 146.875 97.125) (end 146 98) (width 0.2) (layer "F.Cu") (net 6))
 (segment (start 152.5 87) (end 148.5 87) (width 0.2) (layer "F.Cu") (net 6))
 (segment (start 147 70) (end 149.12 67.88) (width 0.2) (layer "F.Cu") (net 6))
 (segment (start 148.5 87) (end 147 85.5) (width 0.2) (layer "F.Cu") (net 6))
 (segment (start 150.375 99.75) (end 150.625 99.75) (width 0.2) (layer "F.Cu") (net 6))
 (segment (start 154.5 102.5) (end 154.5 89) (width 0.2) (layer "F.Cu") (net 6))
 (segment (start 142.125 98) (end 140.375 96.25) (width 0.2) (layer "F.Cu") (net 6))
 (via (at 137 93.5) (size 0.6) (drill 0.3) (layers "F.Cu" "B.Cu") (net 6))
 (via (at 132.5 103) (size 0.6) (drill 0.3) (layers "F.Cu" "B.Cu") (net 6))
 (segment (start 132.5 103) (end 137 98.5) (width 0.2) (layer "B.Cu") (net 6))
 (segment (start 137 98.5) (end 137 93.5) (width 0.2) (layer "B.Cu") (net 6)))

